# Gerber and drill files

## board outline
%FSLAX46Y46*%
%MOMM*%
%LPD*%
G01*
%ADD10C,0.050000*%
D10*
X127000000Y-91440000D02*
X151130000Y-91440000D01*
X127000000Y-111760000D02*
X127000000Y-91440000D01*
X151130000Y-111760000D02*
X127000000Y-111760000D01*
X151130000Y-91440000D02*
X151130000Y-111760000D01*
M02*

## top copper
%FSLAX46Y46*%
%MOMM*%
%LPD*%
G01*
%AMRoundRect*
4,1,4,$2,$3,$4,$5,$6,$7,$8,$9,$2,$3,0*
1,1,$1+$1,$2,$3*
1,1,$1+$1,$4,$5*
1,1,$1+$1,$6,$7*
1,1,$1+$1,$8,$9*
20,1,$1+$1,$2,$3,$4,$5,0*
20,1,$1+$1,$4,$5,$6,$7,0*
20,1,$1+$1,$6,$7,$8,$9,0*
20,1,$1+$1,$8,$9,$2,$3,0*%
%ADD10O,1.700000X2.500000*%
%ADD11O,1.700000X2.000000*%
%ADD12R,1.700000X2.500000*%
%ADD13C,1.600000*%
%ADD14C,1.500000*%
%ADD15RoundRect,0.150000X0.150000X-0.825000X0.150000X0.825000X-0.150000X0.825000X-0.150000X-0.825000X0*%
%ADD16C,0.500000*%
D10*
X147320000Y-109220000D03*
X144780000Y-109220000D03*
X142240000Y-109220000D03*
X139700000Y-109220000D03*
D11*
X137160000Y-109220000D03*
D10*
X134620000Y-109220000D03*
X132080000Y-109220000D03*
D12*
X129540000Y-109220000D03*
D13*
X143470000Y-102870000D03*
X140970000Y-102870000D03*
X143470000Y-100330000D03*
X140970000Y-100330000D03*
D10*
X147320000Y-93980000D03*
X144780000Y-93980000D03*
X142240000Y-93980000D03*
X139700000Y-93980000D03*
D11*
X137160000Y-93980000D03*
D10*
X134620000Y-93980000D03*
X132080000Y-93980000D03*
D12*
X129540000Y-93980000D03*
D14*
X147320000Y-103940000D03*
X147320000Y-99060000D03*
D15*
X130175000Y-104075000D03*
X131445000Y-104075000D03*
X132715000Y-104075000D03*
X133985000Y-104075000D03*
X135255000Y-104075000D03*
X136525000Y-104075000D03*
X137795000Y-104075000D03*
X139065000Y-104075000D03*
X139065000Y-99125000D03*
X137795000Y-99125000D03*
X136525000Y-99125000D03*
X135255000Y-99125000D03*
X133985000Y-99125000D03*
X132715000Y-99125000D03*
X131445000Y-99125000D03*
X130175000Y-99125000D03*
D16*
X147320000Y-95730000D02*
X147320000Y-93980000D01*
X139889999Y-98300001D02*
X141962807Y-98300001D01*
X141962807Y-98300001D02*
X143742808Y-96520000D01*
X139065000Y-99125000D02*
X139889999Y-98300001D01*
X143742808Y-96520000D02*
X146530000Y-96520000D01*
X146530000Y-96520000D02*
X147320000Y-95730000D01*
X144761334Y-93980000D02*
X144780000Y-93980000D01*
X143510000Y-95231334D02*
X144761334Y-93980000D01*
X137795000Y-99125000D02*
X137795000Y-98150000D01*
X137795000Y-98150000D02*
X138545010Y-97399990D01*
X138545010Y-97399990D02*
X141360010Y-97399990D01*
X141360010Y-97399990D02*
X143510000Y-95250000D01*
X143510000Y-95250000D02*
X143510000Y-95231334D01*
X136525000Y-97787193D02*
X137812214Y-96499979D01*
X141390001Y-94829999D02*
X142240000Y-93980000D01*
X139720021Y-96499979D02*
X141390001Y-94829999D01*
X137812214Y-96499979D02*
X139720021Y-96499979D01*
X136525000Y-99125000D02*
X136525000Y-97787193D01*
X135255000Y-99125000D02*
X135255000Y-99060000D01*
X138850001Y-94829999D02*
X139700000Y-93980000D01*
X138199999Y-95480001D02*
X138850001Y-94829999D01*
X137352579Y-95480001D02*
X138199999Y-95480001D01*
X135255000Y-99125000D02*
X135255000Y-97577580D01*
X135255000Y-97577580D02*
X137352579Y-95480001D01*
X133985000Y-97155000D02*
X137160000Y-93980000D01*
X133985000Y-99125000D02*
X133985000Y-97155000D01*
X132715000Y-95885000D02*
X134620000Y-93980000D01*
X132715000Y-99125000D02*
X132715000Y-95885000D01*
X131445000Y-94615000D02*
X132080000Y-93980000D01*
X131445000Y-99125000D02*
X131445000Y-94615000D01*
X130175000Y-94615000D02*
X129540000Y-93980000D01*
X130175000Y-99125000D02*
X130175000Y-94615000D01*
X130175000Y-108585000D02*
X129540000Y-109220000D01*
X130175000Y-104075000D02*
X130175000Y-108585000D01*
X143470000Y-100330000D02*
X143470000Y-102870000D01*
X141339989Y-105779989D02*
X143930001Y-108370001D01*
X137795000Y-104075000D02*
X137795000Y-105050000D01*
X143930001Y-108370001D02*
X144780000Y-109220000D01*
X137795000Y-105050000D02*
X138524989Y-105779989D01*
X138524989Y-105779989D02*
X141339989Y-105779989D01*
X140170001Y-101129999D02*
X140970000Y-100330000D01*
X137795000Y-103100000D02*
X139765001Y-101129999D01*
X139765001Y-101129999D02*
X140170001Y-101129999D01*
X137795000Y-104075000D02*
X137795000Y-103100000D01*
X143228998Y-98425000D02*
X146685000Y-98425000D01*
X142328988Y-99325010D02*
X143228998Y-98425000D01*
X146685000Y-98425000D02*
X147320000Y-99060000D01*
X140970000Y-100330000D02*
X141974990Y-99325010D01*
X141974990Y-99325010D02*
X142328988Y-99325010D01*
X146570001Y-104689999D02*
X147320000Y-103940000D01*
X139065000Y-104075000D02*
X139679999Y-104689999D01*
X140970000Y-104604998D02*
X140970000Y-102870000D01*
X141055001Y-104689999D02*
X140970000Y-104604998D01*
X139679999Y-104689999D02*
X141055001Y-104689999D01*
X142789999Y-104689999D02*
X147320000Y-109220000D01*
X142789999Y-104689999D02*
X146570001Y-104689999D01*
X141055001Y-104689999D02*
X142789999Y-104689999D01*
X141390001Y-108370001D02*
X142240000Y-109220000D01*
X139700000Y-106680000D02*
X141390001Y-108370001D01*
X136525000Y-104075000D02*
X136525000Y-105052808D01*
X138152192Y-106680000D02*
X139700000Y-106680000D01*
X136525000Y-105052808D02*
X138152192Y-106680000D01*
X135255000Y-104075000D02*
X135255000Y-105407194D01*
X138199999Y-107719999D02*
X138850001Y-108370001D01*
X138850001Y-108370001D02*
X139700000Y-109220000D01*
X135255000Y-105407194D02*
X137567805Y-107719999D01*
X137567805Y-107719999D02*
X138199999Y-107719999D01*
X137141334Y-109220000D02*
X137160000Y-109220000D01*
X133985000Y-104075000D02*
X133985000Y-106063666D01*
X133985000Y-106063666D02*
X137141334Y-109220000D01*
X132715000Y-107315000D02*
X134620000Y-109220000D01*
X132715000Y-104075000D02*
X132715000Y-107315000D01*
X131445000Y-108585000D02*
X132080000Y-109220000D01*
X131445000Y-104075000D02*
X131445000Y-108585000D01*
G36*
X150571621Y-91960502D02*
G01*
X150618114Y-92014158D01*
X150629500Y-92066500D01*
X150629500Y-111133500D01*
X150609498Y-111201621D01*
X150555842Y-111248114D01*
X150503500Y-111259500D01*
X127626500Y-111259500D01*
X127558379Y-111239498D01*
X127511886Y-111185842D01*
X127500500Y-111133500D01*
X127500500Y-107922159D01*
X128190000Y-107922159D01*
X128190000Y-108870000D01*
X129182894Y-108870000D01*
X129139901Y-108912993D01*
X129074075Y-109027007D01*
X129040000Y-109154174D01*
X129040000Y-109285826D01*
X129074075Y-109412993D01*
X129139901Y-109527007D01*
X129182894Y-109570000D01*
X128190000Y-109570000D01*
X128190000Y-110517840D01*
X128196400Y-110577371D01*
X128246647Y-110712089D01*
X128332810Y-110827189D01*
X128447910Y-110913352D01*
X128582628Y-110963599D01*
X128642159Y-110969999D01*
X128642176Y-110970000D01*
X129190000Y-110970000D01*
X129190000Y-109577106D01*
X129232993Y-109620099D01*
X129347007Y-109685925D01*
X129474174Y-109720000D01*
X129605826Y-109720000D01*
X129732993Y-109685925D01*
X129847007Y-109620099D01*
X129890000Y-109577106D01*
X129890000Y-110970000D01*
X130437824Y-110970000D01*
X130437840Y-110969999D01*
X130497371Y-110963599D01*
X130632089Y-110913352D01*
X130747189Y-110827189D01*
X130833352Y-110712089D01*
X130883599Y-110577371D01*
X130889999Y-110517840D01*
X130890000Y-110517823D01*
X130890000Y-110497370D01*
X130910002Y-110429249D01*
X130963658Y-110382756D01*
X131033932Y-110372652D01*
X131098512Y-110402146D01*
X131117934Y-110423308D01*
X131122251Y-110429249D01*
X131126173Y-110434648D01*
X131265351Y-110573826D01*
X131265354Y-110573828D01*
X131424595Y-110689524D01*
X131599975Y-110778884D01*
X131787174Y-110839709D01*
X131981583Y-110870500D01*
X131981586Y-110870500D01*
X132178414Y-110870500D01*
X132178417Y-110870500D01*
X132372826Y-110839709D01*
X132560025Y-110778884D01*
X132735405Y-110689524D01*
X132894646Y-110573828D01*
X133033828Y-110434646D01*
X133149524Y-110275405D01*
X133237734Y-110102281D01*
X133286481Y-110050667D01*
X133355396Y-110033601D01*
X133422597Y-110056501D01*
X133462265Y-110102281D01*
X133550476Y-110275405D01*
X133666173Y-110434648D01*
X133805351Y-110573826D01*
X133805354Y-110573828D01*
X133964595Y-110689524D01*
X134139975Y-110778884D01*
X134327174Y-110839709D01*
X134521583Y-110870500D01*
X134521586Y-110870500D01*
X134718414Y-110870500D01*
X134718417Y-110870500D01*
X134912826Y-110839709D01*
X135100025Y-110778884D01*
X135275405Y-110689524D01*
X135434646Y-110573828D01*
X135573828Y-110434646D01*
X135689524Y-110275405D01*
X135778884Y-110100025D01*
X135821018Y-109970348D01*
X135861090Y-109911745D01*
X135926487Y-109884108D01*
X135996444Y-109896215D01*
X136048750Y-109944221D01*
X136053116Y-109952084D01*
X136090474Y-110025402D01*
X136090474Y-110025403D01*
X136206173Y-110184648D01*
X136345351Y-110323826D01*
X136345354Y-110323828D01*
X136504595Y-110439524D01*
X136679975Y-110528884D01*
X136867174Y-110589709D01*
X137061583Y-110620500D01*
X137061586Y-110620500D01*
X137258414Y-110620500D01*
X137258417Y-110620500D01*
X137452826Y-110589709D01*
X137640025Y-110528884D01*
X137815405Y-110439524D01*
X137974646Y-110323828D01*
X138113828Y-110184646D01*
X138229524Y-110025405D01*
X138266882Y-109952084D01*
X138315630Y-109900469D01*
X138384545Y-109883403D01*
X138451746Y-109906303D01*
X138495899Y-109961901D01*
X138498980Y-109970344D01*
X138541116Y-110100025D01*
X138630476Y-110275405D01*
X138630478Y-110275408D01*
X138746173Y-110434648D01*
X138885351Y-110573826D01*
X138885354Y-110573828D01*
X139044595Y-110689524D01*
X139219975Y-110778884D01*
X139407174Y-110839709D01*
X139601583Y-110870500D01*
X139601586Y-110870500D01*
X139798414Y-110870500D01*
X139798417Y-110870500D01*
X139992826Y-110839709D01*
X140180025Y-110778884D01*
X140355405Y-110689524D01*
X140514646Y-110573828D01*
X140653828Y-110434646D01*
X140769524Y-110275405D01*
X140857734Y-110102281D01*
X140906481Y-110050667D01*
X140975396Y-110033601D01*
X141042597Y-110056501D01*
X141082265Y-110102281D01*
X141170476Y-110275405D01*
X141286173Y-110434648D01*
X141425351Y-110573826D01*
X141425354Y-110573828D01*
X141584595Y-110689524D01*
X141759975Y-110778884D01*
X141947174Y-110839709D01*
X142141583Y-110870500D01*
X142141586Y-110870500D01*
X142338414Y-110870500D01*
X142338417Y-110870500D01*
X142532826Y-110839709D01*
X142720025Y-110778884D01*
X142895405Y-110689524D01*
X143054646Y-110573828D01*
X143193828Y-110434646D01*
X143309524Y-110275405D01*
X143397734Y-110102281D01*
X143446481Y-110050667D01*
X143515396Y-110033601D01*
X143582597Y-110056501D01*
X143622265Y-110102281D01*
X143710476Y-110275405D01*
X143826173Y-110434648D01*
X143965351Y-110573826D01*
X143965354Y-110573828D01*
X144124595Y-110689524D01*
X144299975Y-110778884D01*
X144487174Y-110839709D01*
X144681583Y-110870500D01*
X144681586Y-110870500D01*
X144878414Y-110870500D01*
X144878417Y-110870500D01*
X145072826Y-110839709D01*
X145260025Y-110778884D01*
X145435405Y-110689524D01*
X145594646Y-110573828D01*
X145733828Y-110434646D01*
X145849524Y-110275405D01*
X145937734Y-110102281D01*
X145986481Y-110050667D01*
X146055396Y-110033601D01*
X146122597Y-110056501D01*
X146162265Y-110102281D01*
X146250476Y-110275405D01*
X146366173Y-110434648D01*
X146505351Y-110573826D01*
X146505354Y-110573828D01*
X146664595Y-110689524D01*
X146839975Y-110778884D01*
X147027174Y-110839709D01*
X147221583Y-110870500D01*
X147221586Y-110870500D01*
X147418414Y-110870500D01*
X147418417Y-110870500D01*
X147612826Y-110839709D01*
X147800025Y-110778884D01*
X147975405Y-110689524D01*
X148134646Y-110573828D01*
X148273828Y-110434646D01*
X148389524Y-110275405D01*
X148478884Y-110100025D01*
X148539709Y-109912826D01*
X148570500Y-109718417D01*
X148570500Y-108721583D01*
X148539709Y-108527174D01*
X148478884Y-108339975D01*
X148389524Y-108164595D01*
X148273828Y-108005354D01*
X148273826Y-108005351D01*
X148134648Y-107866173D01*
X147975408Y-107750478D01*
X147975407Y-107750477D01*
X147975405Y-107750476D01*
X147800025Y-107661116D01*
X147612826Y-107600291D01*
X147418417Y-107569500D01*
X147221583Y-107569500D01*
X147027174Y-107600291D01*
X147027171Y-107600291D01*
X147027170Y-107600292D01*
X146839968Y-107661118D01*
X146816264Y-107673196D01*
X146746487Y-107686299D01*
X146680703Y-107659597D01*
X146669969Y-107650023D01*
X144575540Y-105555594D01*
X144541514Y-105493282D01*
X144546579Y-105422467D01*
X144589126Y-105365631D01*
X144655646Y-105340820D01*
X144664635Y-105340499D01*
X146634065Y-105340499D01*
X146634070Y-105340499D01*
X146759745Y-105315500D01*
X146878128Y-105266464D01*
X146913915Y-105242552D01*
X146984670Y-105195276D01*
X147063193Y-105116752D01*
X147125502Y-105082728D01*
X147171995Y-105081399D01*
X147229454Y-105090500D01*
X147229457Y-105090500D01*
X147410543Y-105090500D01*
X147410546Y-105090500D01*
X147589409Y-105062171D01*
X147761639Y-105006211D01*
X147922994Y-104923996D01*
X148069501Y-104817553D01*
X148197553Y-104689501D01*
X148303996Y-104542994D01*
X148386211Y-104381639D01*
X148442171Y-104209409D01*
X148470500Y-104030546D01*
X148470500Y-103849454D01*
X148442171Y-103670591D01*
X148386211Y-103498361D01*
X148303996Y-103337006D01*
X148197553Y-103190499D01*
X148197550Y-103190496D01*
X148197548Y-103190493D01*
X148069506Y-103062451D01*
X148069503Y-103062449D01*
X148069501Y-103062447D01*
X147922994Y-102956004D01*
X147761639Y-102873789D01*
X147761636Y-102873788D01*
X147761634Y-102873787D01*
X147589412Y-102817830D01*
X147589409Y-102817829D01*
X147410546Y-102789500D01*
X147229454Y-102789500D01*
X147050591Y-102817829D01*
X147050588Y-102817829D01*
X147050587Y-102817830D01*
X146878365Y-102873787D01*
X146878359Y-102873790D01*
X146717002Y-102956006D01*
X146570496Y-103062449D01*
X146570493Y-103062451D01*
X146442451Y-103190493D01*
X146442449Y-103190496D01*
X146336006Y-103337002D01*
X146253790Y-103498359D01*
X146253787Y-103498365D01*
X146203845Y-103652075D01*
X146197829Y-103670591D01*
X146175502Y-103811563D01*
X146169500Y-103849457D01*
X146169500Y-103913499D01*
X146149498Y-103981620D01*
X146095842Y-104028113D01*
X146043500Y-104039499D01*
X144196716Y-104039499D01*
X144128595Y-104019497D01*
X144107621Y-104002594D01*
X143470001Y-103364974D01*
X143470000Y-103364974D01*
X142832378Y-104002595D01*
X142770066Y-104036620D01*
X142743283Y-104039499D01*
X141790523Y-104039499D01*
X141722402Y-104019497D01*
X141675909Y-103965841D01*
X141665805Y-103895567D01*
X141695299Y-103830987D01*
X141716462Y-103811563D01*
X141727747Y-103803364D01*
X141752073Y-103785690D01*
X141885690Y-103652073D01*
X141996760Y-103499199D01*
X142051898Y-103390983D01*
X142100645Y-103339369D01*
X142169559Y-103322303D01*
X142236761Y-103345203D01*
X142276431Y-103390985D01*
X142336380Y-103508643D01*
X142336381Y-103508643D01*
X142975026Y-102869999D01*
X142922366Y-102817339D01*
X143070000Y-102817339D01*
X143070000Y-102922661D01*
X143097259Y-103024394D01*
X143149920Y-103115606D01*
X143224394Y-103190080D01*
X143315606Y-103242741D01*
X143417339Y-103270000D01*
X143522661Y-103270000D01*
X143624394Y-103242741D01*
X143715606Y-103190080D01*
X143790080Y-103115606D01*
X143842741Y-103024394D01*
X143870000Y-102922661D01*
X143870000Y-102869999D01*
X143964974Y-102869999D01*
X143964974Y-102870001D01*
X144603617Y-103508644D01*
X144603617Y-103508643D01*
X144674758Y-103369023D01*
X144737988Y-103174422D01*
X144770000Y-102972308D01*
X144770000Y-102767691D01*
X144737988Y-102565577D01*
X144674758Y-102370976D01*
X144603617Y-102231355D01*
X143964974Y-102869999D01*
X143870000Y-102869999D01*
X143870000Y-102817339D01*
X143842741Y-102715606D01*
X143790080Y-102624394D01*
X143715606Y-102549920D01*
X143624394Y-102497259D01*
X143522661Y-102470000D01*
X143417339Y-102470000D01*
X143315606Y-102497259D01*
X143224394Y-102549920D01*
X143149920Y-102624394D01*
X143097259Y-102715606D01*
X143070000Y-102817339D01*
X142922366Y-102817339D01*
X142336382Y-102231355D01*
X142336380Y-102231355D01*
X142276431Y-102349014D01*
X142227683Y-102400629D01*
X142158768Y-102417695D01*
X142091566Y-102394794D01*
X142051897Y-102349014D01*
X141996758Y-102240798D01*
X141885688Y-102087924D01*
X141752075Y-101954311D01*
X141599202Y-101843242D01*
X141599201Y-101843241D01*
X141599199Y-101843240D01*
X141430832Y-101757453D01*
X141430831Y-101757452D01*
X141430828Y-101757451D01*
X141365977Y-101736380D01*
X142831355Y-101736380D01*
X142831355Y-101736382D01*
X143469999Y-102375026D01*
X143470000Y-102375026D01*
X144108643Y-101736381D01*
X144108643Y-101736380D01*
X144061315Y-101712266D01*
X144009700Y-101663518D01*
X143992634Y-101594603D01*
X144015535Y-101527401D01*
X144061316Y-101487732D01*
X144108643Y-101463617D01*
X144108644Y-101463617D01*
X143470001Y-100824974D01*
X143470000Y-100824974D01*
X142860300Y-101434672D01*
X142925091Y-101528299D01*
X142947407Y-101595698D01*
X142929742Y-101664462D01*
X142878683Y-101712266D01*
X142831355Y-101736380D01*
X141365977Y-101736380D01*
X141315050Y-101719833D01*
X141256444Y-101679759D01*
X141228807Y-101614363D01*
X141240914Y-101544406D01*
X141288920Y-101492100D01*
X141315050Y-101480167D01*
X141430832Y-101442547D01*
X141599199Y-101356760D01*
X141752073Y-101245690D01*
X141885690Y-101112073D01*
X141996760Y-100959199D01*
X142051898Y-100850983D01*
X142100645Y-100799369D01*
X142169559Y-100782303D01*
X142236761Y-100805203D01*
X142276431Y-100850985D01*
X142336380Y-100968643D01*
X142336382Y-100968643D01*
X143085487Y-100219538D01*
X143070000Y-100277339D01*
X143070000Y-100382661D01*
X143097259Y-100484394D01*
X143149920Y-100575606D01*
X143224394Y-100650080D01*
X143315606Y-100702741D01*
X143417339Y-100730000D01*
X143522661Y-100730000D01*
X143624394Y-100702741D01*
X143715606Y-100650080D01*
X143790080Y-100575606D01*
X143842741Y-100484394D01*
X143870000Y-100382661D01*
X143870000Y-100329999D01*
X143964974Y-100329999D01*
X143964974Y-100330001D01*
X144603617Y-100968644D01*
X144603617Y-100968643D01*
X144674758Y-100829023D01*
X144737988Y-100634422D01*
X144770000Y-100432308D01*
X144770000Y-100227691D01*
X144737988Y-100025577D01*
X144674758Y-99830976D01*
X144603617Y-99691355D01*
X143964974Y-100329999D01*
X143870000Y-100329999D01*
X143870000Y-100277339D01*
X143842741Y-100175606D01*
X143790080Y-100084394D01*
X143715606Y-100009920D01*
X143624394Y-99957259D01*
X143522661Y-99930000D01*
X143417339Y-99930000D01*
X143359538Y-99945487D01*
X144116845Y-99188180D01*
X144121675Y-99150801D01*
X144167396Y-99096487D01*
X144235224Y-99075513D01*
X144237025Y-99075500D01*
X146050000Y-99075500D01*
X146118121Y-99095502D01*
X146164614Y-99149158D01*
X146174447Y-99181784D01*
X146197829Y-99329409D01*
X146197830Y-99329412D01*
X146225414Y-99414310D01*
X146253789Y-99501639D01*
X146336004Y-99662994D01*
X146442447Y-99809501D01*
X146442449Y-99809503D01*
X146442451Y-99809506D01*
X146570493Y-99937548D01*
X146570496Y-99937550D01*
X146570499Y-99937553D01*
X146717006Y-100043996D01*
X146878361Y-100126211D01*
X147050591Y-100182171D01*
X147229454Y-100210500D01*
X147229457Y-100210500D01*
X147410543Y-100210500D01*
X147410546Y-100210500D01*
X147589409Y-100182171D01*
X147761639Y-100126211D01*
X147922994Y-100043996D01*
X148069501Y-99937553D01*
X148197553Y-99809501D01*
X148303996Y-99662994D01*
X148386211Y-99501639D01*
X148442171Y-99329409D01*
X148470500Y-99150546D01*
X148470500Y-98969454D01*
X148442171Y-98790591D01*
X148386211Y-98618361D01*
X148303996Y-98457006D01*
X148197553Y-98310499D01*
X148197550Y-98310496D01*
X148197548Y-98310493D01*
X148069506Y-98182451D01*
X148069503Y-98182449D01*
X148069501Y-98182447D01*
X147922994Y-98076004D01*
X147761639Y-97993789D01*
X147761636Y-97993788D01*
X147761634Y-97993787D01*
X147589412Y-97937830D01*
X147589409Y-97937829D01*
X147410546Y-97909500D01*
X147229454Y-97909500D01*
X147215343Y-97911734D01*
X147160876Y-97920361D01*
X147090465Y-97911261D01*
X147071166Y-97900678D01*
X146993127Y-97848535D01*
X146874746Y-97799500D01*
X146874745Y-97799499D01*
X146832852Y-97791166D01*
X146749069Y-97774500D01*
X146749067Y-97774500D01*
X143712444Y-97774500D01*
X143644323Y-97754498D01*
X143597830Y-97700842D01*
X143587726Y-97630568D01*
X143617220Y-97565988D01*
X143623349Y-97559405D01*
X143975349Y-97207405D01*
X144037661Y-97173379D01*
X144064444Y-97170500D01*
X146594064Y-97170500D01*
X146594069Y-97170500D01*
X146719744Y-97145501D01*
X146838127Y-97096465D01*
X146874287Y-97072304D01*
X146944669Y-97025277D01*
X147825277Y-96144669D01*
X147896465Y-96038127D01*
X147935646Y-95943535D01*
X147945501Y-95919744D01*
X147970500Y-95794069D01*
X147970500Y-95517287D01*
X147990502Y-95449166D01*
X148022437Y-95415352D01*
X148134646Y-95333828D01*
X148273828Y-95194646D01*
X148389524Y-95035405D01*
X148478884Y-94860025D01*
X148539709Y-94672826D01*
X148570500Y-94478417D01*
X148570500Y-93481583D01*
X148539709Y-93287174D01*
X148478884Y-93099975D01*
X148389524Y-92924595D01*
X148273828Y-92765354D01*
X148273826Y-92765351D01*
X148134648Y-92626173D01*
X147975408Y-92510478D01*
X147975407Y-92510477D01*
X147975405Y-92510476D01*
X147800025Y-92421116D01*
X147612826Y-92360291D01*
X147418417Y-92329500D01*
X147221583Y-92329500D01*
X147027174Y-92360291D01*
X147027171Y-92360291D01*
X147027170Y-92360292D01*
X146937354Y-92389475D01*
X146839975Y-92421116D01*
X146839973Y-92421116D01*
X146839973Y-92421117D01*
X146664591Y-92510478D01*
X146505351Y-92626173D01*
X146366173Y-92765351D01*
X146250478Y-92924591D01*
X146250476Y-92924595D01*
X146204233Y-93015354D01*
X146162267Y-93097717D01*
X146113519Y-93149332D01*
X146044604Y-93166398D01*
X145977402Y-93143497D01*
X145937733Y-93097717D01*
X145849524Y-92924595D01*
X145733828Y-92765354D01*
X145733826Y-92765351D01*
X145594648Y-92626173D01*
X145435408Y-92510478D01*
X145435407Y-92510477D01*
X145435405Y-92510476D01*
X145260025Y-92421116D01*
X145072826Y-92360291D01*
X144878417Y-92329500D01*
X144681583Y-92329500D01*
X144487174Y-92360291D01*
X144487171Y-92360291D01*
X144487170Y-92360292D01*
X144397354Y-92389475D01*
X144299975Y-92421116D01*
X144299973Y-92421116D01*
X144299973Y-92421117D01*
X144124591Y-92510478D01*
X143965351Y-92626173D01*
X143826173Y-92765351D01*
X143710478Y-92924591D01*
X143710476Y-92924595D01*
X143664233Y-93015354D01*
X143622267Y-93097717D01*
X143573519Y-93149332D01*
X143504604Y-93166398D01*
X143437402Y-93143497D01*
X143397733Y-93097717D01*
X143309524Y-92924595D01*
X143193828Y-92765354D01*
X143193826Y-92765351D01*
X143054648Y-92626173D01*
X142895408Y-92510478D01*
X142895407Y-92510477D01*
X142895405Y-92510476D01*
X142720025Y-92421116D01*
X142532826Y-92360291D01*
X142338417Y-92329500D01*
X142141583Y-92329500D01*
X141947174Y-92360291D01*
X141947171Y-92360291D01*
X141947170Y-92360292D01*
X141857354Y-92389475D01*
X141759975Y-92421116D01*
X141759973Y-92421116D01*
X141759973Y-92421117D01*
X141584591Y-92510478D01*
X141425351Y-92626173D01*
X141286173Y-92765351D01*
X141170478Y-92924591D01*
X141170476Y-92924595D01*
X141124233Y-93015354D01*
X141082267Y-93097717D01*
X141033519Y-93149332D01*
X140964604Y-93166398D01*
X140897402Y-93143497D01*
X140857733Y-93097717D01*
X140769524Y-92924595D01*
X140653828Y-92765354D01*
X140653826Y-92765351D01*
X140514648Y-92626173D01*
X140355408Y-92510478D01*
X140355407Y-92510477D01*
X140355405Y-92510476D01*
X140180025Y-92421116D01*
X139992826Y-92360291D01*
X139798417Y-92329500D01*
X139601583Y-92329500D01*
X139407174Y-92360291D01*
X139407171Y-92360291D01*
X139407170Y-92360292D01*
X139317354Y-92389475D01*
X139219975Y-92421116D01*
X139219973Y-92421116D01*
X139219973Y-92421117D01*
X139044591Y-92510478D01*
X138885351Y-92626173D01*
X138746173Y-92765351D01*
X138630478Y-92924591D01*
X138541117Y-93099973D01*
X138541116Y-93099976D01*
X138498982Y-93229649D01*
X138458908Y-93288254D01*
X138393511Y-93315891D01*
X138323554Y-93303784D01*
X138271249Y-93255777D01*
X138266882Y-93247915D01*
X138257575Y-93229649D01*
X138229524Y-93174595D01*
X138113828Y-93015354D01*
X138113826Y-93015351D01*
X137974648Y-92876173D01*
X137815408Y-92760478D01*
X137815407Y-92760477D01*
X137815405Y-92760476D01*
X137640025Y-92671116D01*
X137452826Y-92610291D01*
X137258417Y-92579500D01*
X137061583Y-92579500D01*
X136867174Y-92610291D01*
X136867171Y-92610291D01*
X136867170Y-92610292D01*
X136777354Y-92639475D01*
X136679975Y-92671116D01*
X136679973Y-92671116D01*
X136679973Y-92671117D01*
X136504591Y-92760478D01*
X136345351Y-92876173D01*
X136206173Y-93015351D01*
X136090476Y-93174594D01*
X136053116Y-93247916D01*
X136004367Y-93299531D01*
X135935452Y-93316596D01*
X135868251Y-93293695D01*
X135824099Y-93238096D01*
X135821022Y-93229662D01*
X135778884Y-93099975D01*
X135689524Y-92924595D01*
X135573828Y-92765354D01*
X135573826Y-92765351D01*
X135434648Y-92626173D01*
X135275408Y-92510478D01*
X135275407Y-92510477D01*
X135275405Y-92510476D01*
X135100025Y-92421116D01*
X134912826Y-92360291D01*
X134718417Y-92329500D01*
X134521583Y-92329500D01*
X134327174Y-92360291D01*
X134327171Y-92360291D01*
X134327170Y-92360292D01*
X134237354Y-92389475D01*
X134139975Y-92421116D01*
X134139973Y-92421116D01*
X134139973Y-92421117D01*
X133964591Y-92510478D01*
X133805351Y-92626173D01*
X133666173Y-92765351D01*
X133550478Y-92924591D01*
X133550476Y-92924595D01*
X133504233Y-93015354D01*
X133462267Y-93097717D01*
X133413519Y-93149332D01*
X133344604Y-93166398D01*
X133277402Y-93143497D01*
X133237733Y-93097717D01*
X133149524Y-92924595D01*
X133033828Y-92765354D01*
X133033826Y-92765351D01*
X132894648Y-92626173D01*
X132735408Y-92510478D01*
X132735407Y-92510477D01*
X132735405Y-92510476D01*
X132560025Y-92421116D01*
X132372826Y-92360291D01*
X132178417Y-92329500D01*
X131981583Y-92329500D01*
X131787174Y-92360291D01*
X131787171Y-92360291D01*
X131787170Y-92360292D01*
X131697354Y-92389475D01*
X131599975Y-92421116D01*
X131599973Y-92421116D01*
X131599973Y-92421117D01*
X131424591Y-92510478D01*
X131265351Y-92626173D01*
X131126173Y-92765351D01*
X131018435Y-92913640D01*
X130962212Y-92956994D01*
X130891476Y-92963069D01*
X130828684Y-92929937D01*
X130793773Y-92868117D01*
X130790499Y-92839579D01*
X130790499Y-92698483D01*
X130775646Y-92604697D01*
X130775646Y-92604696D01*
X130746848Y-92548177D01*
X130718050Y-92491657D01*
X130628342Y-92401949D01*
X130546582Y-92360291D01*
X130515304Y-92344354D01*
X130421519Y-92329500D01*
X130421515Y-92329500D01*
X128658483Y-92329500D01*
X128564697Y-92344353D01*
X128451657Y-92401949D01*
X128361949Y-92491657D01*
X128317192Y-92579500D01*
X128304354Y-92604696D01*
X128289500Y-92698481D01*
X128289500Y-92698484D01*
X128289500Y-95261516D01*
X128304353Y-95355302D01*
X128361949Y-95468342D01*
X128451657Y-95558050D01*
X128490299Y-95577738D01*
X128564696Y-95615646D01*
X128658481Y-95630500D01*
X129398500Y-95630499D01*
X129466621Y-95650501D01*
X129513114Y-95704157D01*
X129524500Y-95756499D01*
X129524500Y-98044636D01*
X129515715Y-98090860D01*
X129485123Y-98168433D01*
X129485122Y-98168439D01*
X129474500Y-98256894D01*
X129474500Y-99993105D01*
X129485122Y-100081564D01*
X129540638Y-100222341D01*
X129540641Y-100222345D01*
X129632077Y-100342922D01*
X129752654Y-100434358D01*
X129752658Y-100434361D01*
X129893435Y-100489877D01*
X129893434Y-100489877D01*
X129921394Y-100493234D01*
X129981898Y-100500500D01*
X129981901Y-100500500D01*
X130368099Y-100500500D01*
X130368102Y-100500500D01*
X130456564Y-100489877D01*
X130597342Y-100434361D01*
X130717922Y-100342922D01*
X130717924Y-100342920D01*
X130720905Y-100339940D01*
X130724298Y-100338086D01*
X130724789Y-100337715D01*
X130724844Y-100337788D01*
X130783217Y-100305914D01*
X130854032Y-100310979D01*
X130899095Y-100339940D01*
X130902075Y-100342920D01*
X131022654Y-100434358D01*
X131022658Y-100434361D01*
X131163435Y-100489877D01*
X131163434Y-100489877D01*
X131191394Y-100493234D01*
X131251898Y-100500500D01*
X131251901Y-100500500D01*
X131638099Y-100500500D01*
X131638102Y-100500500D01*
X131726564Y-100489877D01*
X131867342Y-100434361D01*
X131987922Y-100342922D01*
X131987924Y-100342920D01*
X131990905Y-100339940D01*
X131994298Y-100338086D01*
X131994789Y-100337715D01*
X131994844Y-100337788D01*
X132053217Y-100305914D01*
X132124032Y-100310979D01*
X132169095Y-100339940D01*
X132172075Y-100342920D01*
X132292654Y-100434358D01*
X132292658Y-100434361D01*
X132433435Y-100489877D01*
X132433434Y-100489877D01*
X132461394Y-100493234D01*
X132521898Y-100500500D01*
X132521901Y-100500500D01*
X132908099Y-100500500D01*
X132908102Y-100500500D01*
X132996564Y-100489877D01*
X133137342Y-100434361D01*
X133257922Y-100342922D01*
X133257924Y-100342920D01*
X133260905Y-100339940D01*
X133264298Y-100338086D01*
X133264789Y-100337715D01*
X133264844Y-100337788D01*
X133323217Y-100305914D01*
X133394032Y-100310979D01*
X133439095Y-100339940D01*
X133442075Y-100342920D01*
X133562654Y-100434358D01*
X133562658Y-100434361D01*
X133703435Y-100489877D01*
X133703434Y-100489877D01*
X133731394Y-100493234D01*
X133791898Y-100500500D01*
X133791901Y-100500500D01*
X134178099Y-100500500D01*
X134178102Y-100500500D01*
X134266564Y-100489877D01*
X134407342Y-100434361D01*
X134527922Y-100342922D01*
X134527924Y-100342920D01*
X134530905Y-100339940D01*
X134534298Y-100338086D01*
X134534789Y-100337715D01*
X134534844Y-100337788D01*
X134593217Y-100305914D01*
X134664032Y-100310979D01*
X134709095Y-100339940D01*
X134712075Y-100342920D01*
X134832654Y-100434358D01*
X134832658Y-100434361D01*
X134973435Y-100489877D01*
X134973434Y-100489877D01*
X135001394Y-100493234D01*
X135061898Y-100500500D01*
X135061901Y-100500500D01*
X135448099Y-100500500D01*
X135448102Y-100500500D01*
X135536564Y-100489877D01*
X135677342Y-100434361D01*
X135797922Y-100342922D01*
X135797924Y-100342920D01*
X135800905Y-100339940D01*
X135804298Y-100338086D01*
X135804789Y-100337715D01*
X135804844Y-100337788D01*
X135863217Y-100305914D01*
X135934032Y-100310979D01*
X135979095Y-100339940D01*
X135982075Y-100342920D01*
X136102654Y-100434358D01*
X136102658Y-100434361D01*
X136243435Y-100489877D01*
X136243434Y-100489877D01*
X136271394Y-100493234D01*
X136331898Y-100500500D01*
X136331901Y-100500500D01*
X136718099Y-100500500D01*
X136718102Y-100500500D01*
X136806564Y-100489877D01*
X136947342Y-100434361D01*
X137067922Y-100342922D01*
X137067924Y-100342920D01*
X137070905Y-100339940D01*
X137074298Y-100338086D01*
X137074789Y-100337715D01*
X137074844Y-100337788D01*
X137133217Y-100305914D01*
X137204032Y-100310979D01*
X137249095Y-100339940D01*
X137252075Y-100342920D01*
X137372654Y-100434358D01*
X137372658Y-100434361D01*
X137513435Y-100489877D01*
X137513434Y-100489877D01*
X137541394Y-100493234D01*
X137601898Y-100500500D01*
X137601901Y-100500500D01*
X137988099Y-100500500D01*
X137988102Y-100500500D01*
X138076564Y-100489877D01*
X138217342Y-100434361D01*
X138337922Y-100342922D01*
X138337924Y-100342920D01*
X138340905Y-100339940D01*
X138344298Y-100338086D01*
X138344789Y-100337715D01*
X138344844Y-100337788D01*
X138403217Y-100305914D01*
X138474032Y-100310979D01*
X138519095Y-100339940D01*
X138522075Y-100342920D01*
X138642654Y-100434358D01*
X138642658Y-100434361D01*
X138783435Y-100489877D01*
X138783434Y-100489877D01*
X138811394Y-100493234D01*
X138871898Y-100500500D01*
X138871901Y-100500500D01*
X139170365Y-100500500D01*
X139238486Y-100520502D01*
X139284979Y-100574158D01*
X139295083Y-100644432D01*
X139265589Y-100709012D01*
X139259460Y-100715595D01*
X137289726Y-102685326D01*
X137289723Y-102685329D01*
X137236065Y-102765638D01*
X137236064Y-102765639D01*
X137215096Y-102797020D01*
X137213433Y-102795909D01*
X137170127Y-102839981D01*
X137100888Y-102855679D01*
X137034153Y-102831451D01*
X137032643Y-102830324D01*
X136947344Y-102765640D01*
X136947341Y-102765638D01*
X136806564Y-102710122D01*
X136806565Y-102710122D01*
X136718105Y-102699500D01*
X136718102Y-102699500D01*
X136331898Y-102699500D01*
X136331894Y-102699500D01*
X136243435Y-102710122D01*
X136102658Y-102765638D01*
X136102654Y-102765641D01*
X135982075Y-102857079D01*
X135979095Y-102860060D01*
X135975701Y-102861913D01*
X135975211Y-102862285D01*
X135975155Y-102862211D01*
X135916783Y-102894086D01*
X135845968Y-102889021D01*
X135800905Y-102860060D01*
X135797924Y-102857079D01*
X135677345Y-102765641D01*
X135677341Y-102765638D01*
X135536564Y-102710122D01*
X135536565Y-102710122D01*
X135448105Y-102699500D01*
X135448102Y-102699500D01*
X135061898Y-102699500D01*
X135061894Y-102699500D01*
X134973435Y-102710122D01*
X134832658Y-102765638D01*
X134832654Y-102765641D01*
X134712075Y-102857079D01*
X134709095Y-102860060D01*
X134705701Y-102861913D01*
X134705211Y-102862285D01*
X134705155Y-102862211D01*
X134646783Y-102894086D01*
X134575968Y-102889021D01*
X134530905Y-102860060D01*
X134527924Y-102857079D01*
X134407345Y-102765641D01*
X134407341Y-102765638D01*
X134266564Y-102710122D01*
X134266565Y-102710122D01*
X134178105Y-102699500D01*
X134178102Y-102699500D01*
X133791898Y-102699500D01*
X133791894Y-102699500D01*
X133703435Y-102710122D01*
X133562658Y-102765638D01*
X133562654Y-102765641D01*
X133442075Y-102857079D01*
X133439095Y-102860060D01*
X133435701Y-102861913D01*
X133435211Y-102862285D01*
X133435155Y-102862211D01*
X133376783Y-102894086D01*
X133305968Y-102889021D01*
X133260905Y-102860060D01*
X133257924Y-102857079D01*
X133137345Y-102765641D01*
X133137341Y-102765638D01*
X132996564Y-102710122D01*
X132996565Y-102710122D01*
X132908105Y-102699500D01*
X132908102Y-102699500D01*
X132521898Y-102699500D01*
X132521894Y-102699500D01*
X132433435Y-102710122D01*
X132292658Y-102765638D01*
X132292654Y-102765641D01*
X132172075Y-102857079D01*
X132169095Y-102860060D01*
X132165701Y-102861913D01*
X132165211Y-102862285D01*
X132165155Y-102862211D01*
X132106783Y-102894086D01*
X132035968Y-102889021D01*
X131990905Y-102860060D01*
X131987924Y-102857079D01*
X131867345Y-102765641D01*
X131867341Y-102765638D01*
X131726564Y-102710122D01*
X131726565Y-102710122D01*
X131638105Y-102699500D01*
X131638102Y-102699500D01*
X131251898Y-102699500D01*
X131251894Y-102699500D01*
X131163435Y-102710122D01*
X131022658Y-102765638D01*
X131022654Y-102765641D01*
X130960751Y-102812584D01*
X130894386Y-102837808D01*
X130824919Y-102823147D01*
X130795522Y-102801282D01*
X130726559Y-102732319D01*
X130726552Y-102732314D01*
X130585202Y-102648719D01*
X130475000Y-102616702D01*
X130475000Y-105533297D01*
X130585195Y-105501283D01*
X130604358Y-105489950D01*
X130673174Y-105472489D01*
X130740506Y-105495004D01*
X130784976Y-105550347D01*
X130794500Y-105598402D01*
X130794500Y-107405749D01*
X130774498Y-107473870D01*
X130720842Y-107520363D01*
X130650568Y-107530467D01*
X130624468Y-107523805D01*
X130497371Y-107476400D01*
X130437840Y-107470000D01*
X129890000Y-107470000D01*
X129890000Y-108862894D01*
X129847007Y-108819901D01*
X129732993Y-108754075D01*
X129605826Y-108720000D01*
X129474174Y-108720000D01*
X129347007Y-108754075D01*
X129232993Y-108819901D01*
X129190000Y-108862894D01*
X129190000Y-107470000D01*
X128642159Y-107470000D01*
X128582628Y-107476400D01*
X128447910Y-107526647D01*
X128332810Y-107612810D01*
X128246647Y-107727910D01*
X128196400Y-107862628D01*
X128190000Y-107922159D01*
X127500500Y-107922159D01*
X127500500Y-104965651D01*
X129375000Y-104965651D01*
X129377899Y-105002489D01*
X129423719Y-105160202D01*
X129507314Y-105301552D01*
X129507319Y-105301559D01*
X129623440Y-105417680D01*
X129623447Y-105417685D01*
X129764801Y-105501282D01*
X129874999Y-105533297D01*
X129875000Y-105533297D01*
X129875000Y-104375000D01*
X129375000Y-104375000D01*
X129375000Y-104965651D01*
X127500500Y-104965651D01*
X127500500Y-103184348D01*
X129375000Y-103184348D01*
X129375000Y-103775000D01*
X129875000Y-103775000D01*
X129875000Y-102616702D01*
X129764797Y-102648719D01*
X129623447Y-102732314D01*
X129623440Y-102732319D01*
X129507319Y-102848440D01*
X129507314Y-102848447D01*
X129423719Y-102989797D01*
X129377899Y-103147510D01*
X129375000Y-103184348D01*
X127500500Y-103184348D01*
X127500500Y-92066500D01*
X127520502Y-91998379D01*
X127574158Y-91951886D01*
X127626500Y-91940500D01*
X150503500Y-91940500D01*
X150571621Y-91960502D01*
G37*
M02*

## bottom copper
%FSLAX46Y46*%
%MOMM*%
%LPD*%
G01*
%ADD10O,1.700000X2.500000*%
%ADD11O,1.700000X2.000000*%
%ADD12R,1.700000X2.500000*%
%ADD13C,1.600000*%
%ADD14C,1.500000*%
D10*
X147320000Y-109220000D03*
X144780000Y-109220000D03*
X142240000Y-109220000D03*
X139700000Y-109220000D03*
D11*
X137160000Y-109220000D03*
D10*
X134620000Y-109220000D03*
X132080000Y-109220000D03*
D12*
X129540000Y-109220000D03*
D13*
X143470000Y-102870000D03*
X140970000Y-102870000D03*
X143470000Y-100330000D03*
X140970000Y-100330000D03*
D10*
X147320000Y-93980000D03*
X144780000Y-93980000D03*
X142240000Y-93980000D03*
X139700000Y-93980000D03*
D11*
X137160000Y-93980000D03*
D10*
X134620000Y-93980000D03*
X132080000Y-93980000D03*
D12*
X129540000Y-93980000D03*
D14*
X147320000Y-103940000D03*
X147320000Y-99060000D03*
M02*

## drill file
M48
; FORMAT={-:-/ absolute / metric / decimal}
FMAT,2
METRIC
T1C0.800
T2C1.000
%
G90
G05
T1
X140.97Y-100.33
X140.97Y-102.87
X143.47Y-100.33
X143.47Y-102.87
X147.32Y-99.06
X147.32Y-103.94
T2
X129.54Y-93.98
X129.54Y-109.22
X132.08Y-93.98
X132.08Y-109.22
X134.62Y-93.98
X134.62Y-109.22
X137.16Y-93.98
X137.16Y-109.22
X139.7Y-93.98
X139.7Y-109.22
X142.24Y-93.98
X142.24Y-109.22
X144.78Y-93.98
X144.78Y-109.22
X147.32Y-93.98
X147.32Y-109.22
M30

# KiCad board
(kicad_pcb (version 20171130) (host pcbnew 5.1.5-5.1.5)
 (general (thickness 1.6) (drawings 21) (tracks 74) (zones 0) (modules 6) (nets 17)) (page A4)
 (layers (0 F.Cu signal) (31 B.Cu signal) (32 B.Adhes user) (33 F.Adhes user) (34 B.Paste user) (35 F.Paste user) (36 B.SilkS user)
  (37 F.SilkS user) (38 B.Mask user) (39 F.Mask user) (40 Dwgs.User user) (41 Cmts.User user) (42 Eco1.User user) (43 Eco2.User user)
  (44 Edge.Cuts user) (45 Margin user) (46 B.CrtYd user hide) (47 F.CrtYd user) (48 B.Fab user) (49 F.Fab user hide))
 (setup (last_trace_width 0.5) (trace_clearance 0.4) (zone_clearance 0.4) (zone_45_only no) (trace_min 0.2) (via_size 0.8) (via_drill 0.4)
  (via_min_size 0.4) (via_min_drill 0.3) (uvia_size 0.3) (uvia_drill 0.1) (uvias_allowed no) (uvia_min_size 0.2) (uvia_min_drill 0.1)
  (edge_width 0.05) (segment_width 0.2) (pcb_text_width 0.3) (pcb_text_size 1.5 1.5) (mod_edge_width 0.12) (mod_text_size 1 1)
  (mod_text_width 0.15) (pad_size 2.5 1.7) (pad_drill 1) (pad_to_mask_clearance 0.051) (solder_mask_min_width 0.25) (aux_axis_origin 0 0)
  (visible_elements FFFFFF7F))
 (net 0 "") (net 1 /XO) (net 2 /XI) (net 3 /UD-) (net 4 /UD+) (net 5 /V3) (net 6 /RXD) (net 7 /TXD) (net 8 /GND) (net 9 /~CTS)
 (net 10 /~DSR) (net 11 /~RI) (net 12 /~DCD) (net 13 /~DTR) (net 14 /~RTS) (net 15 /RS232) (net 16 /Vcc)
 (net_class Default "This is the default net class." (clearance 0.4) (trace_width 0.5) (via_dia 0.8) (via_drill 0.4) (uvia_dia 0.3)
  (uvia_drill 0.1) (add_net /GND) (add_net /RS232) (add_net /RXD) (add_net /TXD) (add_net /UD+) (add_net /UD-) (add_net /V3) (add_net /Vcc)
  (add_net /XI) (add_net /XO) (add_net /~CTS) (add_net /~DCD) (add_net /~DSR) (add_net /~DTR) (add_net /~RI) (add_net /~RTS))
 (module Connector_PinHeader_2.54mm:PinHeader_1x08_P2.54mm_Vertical (layer B.Cu) (at 129.54 109.22 270)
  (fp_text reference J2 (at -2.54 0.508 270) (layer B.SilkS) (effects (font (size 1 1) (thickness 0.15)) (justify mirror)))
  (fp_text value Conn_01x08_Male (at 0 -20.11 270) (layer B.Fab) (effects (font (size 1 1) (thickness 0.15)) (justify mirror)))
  (pad 8 thru_hole oval (at 0 -17.78 270) (size 2.5 1.7) (drill 1) (layers *.Cu *.Mask) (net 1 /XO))
  (pad 7 thru_hole oval (at 0 -15.24 270) (size 2.5 1.7) (drill 1) (layers *.Cu *.Mask) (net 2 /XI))
  (pad 6 thru_hole oval (at 0 -12.7 270) (size 2.5 1.7) (drill 1) (layers *.Cu *.Mask) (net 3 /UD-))
  (pad 5 thru_hole oval (at 0 -10.16 270) (size 2.5 1.7) (drill 1) (layers *.Cu *.Mask) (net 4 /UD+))
  (pad 4 thru_hole oval (at 0 -7.62 270) (size 2 1.7) (drill 1) (layers *.Cu *.Mask) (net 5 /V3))
  (pad 3 thru_hole oval (at 0 -5.08 270) (size 2.5 1.7) (drill 1) (layers *.Cu *.Mask) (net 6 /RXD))
  (pad 2 thru_hole oval (at 0 -2.54 270) (size 2.5 1.7) (drill 1) (layers *.Cu *.Mask) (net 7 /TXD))
  (pad 1 thru_hole rect (at 0 0 270) (size 2.5 1.7) (drill 1) (layers *.Cu *.Mask) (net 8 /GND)))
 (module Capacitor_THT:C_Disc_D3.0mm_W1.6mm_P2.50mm (layer F.Cu) (at 140.97 102.87)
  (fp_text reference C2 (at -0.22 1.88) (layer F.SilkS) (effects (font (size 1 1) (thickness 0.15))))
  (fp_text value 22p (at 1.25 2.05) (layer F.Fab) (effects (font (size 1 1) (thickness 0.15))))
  (pad 2 thru_hole circle (at 2.5 0) (size 1.6 1.6) (drill 0.8) (layers *.Cu *.Mask) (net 8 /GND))
  (pad 1 thru_hole circle (at 0 0) (size 1.6 1.6) (drill 0.8) (layers *.Cu *.Mask) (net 1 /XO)))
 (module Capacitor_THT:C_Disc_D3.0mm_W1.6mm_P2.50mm (layer F.Cu) (at 140.97 100.33)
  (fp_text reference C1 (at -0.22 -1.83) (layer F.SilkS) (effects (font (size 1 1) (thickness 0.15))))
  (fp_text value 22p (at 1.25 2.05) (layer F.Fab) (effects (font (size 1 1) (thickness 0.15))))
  (pad 2 thru_hole circle (at 2.5 0) (size 1.6 1.6) (drill 0.8) (layers *.Cu *.Mask) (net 8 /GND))
  (pad 1 thru_hole circle (at 0 0) (size 1.6 1.6) (drill 0.8) (layers *.Cu *.Mask) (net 2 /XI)))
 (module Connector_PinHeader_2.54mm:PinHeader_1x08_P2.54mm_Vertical (layer B.Cu) (at 129.54 93.98 270)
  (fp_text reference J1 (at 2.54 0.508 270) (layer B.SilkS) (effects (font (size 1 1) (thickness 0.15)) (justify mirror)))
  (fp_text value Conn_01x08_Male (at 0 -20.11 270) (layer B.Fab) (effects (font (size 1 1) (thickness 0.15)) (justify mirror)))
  (pad 8 thru_hole oval (at 0 -17.78 270) (size 2.5 1.7) (drill 1) (layers *.Cu *.Mask) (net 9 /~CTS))
  (pad 7 thru_hole oval (at 0 -15.24 270) (size 2.5 1.7) (drill 1) (layers *.Cu *.Mask) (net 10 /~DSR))
  (pad 6 thru_hole oval (at 0 -12.7 270) (size 2.5 1.7) (drill 1) (layers *.Cu *.Mask) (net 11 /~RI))
  (pad 5 thru_hole oval (at 0 -10.16 270) (size 2.5 1.7) (drill 1) (layers *.Cu *.Mask) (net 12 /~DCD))
  (pad 4 thru_hole oval (at 0 -7.62 270) (size 2 1.7) (drill 1) (layers *.Cu *.Mask) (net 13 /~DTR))
  (pad 3 thru_hole oval (at 0 -5.08 270) (size 2.5 1.7) (drill 1) (layers *.Cu *.Mask) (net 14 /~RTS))
  (pad 2 thru_hole oval (at 0 -2.54 270) (size 2.5 1.7) (drill 1) (layers *.Cu *.Mask) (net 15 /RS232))
  (pad 1 thru_hole rect (at 0 0 270) (size 2.5 1.7) (drill 1) (layers *.Cu *.Mask) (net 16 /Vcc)))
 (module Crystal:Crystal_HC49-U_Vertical (layer F.Cu) (at 147.32 99.06 270)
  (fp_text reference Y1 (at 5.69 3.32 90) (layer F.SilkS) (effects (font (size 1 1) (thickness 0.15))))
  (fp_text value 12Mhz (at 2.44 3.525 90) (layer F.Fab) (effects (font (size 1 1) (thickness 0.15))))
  (pad 2 thru_hole circle (at 4.88 0 270) (size 1.5 1.5) (drill 0.8) (layers *.Cu *.Mask) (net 1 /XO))
  (pad 1 thru_hole circle (at 0 0 270) (size 1.5 1.5) (drill 0.8) (layers *.Cu *.Mask) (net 2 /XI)))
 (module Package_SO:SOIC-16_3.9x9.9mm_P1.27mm (layer F.Cu) (at 134.62 101.6 90)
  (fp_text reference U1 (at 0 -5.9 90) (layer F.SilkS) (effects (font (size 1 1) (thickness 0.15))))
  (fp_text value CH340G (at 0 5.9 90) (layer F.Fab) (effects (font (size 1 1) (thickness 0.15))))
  (pad 1 smd roundrect (at -2.475 -4.445 90) (size 1.95 0.6) (layers F.Cu F.Paste F.Mask) (roundrect_rratio 0.25) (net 8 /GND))
  (pad 2 smd roundrect (at -2.475 -3.175 90) (size 1.95 0.6) (layers F.Cu F.Paste F.Mask) (roundrect_rratio 0.25) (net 7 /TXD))
  (pad 3 smd roundrect (at -2.475 -1.905 90) (size 1.95 0.6) (layers F.Cu F.Paste F.Mask) (roundrect_rratio 0.25) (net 6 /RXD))
  (pad 4 smd roundrect (at -2.475 -0.635 90) (size 1.95 0.6) (layers F.Cu F.Paste F.Mask) (roundrect_rratio 0.25) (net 5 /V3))
  (pad 5 smd roundrect (at -2.475 0.635 90) (size 1.95 0.6) (layers F.Cu F.Paste F.Mask) (roundrect_rratio 0.25) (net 4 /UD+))
  (pad 6 smd roundrect (at -2.475 1.905 90) (size 1.95 0.6) (layers F.Cu F.Paste F.Mask) (roundrect_rratio 0.25) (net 3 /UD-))
  (pad 7 smd roundrect (at -2.475 3.175 90) (size 1.95 0.6) (layers F.Cu F.Paste F.Mask) (roundrect_rratio 0.25) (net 2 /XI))
  (pad 8 smd roundrect (at -2.475 4.445 90) (size 1.95 0.6) (layers F.Cu F.Paste F.Mask) (roundrect_rratio 0.25) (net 1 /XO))
  (pad 9 smd roundrect (at 2.475 4.445 90) (size 1.95 0.6) (layers F.Cu F.Paste F.Mask) (roundrect_rratio 0.25) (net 9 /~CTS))
  (pad 10 smd roundrect (at 2.475 3.175 90) (size 1.95 0.6) (layers F.Cu F.Paste F.Mask) (roundrect_rratio 0.25) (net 10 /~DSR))
  (pad 11 smd roundrect (at 2.475 1.905 90) (size 1.95 0.6) (layers F.Cu F.Paste F.Mask) (roundrect_rratio 0.25) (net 11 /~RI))
  (pad 12 smd roundrect (at 2.475 0.635 90) (size 1.95 0.6) (layers F.Cu F.Paste F.Mask) (roundrect_rratio 0.25) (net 12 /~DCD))
  (pad 13 smd roundrect (at 2.475 -0.635 90) (size 1.95 0.6) (layers F.Cu F.Paste F.Mask) (roundrect_rratio 0.25) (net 13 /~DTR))
  (pad 14 smd roundrect (at 2.475 -1.905 90) (size 1.95 0.6) (layers F.Cu F.Paste F.Mask) (roundrect_rratio 0.25) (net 14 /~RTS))
  (pad 15 smd roundrect (at 2.475 -3.175 90) (size 1.95 0.6) (layers F.Cu F.Paste F.Mask) (roundrect_rratio 0.25) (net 15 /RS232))
  (pad 16 smd roundrect (at 2.475 -4.445 90) (size 1.95 0.6) (layers F.Cu F.Paste F.Mask) (roundrect_rratio 0.25) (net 16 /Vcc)))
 (gr_line (start 127 91.44) (end 151.13 91.44) (layer Edge.Cuts) (width 0.05))
 (gr_line (start 127 111.76) (end 127 91.44) (layer Edge.Cuts) (width 0.05))
 (gr_line (start 151.13 111.76) (end 127 111.76) (layer Edge.Cuts) (width 0.05))
 (gr_line (start 151.13 91.44) (end 151.13 111.76) (layer Edge.Cuts) (width 0.05))
 (segment (start 147.32 95.73) (end 147.32 93.98) (width 0.5) (layer F.Cu) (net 9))
 (segment (start 139.889999 98.300001) (end 141.962807 98.300001) (width 0.5) (layer F.Cu) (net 9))
 (segment (start 141.962807 98.300001) (end 143.742808 96.52) (width 0.5) (layer F.Cu) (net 9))
 (segment (start 139.065 99.125) (end 139.889999 98.300001) (width 0.5) (layer F.Cu) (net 9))
 (segment (start 143.742808 96.52) (end 146.53 96.52) (width 0.5) (layer F.Cu) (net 9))
 (segment (start 146.53 96.52) (end 147.32 95.73) (width 0.5) (layer F.Cu) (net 9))
 (segment (start 144.761334 93.98) (end 144.78 93.98) (width 0.5) (layer F.Cu) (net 10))
 (segment (start 143.51 95.231334) (end 144.761334 93.98) (width 0.5) (layer F.Cu) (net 10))
 (segment (start 137.795 99.125) (end 137.795 98.15) (width 0.5) (layer F.Cu) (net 10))
 (segment (start 137.795 98.15) (end 138.54501 97.39999) (width 0.5) (layer F.Cu) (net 10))
 (segment (start 138.54501 97.39999) (end 141.36001 97.39999) (width 0.5) (layer F.Cu) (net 10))
 (segment (start 141.36001 97.39999) (end 143.51 95.25) (width 0.5) (layer F.Cu) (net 10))
 (segment (start 143.51 95.25) (end 143.51 95.231334) (width 0.5) (layer F.Cu) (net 10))
 (segment (start 136.525 97.787193) (end 137.812214 96.499979) (width 0.5) (layer F.Cu) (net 11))
 (segment (start 141.390001 94.829999) (end 142.24 93.98) (width 0.5) (layer F.Cu) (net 11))
 (segment (start 139.720021 96.499979) (end 141.390001 94.829999) (width 0.5) (layer F.Cu) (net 11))
 (segment (start 137.812214 96.499979) (end 139.720021 96.499979) (width 0.5) (layer F.Cu) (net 11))
 (segment (start 136.525 99.125) (end 136.525 97.787193) (width 0.5) (layer F.Cu) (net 11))
 (segment (start 135.255 99.125) (end 135.255 99.06) (width 0.5) (layer F.Cu) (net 12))
 (segment (start 138.850001 94.829999) (end 139.7 93.98) (width 0.5) (layer F.Cu) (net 12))
 (segment (start 138.199999 95.480001) (end 138.850001 94.829999) (width 0.5) (layer F.Cu) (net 12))
 (segment (start 137.352579 95.480001) (end 138.199999 95.480001) (width 0.5) (layer F.Cu) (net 12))
 (segment (start 135.255 99.125) (end 135.255 97.57758) (width 0.5) (layer F.Cu) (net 12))
 (segment (start 135.255 97.57758) (end 137.352579 95.480001) (width 0.5) (layer F.Cu) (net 12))
 (segment (start 133.985 97.155) (end 137.16 93.98) (width 0.5) (layer F.Cu) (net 13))
 (segment (start 133.985 99.125) (end 133.985 97.155) (width 0.5) (layer F.Cu) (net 13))
 (segment (start 132.715 95.885) (end 134.62 93.98) (width 0.5) (layer F.Cu) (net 14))
 (segment (start 132.715 99.125) (end 132.715 95.885) (width 0.5) (layer F.Cu) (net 14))
 (segment (start 131.445 94.615) (end 132.08 93.98) (width 0.5) (layer F.Cu) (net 15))
 (segment (start 131.445 99.125) (end 131.445 94.615) (width 0.5) (layer F.Cu) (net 15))
 (segment (start 130.175 94.615) (end 129.54 93.98) (width 0.5) (layer F.Cu) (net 16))
 (segment (start 130.175 99.125) (end 130.175 94.615) (width 0.5) (layer F.Cu) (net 16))
 (segment (start 130.175 108.585) (end 129.54 109.22) (width 0.5) (layer F.Cu) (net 8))
 (segment (start 130.175 104.075) (end 130.175 108.585) (width 0.5) (layer F.Cu) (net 8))
 (segment (start 143.47 100.33) (end 143.47 102.87) (width 0.5) (layer F.Cu) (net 8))
 (segment (start 141.339989 105.779989) (end 143.930001 108.370001) (width 0.5) (layer F.Cu) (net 2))
 (segment (start 137.795 104.075) (end 137.795 105.05) (width 0.5) (layer F.Cu) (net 2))
 (segment (start 143.930001 108.370001) (end 144.78 109.22) (width 0.5) (layer F.Cu) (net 2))
 (segment (start 137.795 105.05) (end 138.524989 105.779989) (width 0.5) (layer F.Cu) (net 2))
 (segment (start 138.524989 105.779989) (end 141.339989 105.779989) (width 0.5) (layer F.Cu) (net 2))
 (segment (start 140.170001 101.129999) (end 140.97 100.33) (width 0.5) (layer F.Cu) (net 2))
 (segment (start 137.795 103.1) (end 139.765001 101.129999) (width 0.5) (layer F.Cu) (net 2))
 (segment (start 139.765001 101.129999) (end 140.170001 101.129999) (width 0.5) (layer F.Cu) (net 2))
 (segment (start 137.795 104.075) (end 137.795 103.1) (width 0.5) (layer F.Cu) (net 2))
 (segment (start 143.228998 98.425) (end 146.685 98.425) (width 0.5) (layer F.Cu) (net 2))
 (segment (start 142.328988 99.32501) (end 143.228998 98.425) (width 0.5) (layer F.Cu) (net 2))
 (segment (start 146.685 98.425) (end 147.32 99.06) (width 0.5) (layer F.Cu) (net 2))
 (segment (start 140.97 100.33) (end 141.97499 99.32501) (width 0.5) (layer F.Cu) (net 2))
 (segment (start 141.97499 99.32501) (end 142.328988 99.32501) (width 0.5) (layer F.Cu) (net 2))
 (segment (start 146.570001 104.689999) (end 147.32 103.94) (width 0.5) (layer F.Cu) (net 1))
 (segment (start 139.065 104.075) (end 139.679999 104.689999) (width 0.5) (layer F.Cu) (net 1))
 (segment (start 140.97 104.604998) (end 140.97 102.87) (width 0.5) (layer F.Cu) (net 1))
 (segment (start 141.055001 104.689999) (end 140.97 104.604998) (width 0.5) (layer F.Cu) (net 1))
 (segment (start 139.679999 104.689999) (end 141.055001 104.689999) (width 0.5) (layer F.Cu) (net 1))
 (segment (start 142.789999 104.689999) (end 147.32 109.22) (width 0.5) (layer F.Cu) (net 1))
 (segment (start 142.789999 104.689999) (end 146.570001 104.689999) (width 0.5) (layer F.Cu) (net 1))
 (segment (start 141.055001 104.689999) (end 142.789999 104.689999) (width 0.5) (layer F.Cu) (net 1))
 (segment (start 141.390001 108.370001) (end 142.24 109.22) (width 0.5) (layer F.Cu) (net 3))
 (segment (start 139.7 106.68) (end 141.390001 108.370001) (width 0.5) (layer F.Cu) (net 3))
 (segment (start 136.525 104.075) (end 136.525 105.052808) (width 0.5) (layer F.Cu) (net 3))
 (segment (start 138.152192 106.68) (end 139.7 106.68) (width 0.5) (layer F.Cu) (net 3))
 (segment (start 136.525 105.052808) (end 138.152192 106.68) (width 0.5) (layer F.Cu) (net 3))
 (segment (start 135.255 104.075) (end 135.255 105.407194) (width 0.5) (layer F.Cu) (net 4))
 (segment (start 138.199999 107.719999) (end 138.850001 108.370001) (width 0.5) (layer F.Cu) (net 4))
 (segment (start 138.850001 108.370001) (end 139.7 109.22) (width 0.5) (layer F.Cu) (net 4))
 (segment (start 135.255 105.407194) (end 137.567805 107.719999) (width 0.5) (layer F.Cu) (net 4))
 (segment (start 137.567805 107.719999) (end 138.199999 107.719999) (width 0.5) (layer F.Cu) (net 4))
 (segment (start 137.141334 109.22) (end 137.16 109.22) (width 0.5) (layer F.Cu) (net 5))
 (segment (start 133.985 104.075) (end 133.985 106.063666) (width 0.5) (layer F.Cu) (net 5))
 (segment (start 133.985 106.063666) (end 137.141334 109.22) (width 0.5) (layer F.Cu) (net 5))
 (segment (start 132.715 107.315) (end 134.62 109.22) (width 0.5) (layer F.Cu) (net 6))
 (segment (start 132.715 104.075) (end 132.715 107.315) (width 0.5) (layer F.Cu) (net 6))
 (segment (start 131.445 108.585) (end 132.08 109.22) (width 0.5) (layer F.Cu) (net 7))
 (segment (start 131.445 104.075) (end 131.445 108.585) (width 0.5) (layer F.Cu) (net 7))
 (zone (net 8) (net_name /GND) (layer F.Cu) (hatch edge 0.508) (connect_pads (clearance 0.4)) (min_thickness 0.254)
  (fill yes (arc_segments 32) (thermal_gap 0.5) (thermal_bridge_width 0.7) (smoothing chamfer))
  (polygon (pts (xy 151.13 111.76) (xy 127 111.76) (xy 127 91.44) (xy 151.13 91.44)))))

